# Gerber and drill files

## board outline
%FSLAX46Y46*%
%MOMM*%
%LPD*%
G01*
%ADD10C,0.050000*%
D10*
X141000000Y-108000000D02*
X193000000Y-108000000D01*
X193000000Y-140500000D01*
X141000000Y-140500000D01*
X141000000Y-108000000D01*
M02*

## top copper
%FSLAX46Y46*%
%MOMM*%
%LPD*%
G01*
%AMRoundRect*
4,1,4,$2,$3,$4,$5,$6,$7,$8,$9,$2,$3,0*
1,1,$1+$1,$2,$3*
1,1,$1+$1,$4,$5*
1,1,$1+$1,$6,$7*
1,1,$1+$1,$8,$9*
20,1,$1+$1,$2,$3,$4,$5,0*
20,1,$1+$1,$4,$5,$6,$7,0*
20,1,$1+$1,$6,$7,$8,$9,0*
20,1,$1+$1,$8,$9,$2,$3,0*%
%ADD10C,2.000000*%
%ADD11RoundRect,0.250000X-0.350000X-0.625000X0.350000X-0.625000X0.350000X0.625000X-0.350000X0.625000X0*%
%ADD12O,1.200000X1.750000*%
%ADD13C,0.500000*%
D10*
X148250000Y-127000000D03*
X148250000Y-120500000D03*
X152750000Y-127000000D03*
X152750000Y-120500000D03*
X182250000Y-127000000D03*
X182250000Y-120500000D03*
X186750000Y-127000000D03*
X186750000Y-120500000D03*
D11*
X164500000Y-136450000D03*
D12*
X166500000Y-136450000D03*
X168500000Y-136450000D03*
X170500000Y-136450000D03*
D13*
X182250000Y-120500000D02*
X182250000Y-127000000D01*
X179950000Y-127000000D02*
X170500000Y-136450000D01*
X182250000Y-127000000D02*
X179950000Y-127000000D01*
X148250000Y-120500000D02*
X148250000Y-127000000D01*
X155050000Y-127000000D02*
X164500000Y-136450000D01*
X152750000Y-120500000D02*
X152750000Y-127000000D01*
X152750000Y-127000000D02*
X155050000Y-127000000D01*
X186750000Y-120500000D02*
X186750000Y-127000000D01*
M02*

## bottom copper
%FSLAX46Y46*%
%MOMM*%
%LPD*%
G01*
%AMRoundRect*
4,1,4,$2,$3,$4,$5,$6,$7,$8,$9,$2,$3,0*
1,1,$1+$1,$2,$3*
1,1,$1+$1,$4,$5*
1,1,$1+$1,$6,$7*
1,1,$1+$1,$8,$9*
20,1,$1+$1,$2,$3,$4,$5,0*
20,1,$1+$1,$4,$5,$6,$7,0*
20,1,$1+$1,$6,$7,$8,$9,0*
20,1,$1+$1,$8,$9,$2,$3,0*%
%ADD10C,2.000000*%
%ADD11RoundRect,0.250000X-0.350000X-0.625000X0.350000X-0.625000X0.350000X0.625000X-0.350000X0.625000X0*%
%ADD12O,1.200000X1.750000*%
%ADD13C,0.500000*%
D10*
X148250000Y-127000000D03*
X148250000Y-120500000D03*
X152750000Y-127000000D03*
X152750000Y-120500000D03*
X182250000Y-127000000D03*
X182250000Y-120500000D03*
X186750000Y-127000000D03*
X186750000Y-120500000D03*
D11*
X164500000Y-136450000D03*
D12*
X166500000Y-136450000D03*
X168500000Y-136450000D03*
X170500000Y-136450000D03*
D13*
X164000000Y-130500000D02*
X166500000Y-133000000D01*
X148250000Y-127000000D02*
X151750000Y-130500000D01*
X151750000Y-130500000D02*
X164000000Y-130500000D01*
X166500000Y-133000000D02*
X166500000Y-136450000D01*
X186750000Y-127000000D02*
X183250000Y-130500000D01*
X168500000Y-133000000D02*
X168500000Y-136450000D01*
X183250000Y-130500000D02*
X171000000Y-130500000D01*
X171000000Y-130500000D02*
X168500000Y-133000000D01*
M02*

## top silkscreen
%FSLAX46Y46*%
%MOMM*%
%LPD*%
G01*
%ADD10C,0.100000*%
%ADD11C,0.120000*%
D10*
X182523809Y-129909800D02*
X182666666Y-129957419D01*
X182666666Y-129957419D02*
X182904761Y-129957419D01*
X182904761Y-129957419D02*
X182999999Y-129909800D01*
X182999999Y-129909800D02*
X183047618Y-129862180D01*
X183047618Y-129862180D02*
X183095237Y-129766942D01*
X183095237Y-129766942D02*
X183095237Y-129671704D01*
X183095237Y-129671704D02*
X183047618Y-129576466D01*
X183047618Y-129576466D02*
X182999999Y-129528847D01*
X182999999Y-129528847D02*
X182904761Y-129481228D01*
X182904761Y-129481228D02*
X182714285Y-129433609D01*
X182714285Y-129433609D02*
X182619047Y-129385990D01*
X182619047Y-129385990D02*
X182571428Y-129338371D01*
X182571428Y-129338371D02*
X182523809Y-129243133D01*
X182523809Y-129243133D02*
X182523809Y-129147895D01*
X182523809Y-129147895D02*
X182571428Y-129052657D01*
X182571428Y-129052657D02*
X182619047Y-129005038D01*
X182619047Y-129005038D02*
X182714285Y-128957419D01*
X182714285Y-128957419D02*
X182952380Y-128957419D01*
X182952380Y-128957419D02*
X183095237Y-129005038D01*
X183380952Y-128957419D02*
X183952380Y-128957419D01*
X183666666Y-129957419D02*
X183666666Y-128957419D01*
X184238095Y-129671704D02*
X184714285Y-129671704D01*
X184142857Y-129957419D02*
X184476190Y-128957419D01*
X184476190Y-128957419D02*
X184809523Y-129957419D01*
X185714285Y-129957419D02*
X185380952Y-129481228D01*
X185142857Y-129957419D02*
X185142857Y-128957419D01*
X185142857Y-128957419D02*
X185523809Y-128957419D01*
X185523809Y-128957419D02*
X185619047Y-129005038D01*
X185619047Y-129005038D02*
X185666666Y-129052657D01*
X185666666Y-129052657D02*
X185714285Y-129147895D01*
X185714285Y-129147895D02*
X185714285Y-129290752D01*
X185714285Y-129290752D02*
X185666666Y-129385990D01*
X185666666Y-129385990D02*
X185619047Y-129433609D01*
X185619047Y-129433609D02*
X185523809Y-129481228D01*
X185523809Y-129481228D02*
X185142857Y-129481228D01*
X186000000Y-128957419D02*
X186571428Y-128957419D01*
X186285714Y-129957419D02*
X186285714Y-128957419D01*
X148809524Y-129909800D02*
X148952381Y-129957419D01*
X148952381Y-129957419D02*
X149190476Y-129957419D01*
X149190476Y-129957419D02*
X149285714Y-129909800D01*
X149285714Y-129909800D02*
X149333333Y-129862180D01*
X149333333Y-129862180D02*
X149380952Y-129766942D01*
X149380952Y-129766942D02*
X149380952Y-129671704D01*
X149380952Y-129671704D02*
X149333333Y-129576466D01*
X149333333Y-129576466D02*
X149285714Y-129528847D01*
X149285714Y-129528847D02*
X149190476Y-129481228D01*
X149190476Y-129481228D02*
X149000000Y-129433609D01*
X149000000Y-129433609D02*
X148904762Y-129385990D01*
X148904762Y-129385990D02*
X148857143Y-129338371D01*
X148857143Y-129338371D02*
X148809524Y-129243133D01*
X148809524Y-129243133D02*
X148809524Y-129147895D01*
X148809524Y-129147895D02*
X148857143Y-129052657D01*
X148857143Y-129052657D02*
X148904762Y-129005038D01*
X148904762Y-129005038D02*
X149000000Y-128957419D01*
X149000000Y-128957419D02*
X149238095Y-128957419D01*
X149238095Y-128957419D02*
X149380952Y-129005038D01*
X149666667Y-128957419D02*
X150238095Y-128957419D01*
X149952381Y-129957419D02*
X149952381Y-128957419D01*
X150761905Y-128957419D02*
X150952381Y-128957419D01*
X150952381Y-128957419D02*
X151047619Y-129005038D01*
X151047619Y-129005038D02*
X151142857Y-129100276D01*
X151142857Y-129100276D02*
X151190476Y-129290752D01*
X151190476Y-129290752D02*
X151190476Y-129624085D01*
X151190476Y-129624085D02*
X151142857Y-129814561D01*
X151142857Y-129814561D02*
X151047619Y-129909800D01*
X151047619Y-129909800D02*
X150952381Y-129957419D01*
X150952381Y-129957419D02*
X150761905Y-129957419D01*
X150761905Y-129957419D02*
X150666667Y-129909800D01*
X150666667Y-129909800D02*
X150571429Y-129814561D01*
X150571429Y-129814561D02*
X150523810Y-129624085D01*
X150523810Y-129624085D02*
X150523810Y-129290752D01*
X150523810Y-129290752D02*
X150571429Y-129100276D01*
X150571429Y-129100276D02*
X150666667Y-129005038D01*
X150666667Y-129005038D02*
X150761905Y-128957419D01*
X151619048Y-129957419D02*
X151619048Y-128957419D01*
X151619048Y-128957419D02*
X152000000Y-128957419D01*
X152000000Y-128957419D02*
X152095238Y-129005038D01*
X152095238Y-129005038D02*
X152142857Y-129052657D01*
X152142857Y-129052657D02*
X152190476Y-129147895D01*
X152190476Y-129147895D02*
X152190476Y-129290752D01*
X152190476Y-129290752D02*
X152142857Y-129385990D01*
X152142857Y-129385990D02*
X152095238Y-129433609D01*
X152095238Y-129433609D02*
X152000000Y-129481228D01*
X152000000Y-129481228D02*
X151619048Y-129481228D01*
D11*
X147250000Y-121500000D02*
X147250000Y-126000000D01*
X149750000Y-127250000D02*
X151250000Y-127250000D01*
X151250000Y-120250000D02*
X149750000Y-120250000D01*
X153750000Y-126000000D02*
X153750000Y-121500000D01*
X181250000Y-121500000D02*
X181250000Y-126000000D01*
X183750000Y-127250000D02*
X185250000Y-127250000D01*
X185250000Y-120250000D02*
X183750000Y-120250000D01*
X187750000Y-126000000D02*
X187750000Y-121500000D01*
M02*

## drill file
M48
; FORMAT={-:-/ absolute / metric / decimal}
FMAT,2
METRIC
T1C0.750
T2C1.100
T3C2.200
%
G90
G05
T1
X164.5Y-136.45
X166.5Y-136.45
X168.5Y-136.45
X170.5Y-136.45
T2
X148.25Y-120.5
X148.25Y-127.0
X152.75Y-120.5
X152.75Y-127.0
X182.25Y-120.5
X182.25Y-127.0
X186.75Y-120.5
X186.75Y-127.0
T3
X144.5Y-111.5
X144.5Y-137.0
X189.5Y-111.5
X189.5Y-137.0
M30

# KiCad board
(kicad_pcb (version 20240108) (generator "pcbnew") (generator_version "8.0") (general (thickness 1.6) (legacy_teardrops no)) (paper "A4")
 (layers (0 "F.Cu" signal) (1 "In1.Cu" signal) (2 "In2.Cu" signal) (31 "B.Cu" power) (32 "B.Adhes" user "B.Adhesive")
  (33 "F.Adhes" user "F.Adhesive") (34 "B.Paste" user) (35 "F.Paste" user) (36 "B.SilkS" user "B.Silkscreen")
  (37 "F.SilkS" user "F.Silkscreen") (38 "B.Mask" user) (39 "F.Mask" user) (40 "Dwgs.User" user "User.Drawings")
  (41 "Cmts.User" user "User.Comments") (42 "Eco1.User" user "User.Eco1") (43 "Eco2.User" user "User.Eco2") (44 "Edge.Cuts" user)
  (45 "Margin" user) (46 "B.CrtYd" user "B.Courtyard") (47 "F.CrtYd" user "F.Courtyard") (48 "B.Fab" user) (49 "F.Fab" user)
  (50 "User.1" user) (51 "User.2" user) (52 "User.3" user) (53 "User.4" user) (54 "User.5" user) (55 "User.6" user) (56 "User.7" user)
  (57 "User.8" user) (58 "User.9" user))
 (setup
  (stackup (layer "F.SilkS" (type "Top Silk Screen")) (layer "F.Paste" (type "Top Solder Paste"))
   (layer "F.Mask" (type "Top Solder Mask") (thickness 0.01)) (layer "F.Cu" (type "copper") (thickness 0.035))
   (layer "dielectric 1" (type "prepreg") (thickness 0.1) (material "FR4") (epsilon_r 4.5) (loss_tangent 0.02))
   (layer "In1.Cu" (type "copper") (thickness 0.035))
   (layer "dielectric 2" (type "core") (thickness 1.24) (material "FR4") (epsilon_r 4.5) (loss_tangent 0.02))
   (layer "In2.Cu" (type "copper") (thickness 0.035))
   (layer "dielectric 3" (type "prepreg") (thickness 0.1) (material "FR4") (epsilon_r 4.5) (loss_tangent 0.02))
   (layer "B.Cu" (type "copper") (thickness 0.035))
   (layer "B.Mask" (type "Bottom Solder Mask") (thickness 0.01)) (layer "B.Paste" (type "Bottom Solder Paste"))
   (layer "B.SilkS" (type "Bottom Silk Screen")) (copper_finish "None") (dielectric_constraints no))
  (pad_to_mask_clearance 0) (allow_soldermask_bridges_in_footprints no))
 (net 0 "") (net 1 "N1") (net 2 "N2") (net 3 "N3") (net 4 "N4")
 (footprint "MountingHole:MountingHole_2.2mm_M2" (layer "F.Cu") (at 144.5 137)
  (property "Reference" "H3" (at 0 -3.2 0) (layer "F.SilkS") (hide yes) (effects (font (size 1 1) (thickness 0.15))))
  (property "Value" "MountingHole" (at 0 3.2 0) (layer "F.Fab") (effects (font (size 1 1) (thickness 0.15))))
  (pad "" np_thru_hole circle (at 0 0) (size 2.2 2.2) (drill 2.2) (layers "*.Cu" "*.Mask")))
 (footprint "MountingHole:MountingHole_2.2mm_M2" (layer "F.Cu") (at 189.5 137)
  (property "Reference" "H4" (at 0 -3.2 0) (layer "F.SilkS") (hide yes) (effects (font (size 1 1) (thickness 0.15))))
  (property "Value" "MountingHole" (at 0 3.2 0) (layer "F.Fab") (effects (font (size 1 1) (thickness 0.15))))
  (pad "" np_thru_hole circle (at 0 0) (size 2.2 2.2) (drill 2.2) (layers "*.Cu" "*.Mask")))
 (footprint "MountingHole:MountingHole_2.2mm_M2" (layer "F.Cu") (at 189.5 111.5)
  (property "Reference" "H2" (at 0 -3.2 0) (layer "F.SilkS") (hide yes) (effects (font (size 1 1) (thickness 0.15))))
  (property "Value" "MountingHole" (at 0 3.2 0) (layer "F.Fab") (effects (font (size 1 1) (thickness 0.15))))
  (pad "" np_thru_hole circle (at 0 0) (size 2.2 2.2) (drill 2.2) (layers "*.Cu" "*.Mask")))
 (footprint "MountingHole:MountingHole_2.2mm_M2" (layer "F.Cu") (at 144.5 111.5)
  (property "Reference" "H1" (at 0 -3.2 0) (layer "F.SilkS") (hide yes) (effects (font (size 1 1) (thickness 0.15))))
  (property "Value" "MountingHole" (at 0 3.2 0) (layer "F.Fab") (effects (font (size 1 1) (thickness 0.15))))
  (pad "" np_thru_hole circle (at 0 0) (size 2.2 2.2) (drill 2.2) (layers "*.Cu" "*.Mask")))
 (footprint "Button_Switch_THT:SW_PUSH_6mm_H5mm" (layer "F.Cu") (at 148.25 127 90)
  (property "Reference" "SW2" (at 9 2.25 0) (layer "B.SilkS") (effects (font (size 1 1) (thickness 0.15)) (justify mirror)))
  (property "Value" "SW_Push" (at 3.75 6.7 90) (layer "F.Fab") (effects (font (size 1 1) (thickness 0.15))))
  (fp_line (start 5.5 -1) (end 1 -1) (stroke (width 0.12) (type solid)) (layer "F.SilkS"))
  (fp_line (start -0.25 1.5) (end -0.25 3) (stroke (width 0.12) (type solid)) (layer "F.SilkS"))
  (fp_line (start 6.75 3) (end 6.75 1.5) (stroke (width 0.12) (type solid)) (layer "F.SilkS"))
  (fp_line (start 1 5.5) (end 5.5 5.5) (stroke (width 0.12) (type solid)) (layer "F.SilkS"))
  (pad "1" thru_hole circle (at 0 0 180) (size 2 2) (drill 1.1) (layers "*.Cu" "*.Mask") (remove_unused_layers no) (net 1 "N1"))
  (pad "1" thru_hole circle (at 6.5 0 180) (size 2 2) (drill 1.1) (layers "*.Cu" "*.Mask") (remove_unused_layers no) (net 1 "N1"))
  (pad "2" thru_hole circle (at 0 4.5 180) (size 2 2) (drill 1.1) (layers "*.Cu" "*.Mask") (remove_unused_layers no) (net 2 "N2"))
  (pad "2" thru_hole circle (at 6.5 4.5 180) (size 2 2) (drill 1.1) (layers "*.Cu" "*.Mask") (remove_unused_layers no) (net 2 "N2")))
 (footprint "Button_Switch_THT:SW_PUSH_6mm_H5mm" (layer "F.Cu") (at 182.25 127 90)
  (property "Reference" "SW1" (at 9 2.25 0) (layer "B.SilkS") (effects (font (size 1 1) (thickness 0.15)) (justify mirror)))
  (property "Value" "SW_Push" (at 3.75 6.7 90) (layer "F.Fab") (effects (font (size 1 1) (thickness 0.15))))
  (fp_line (start 5.5 -1) (end 1 -1) (stroke (width 0.12) (type solid)) (layer "F.SilkS"))
  (fp_line (start -0.25 1.5) (end -0.25 3) (stroke (width 0.12) (type solid)) (layer "F.SilkS"))
  (fp_line (start 6.75 3) (end 6.75 1.5) (stroke (width 0.12) (type solid)) (layer "F.SilkS"))
  (fp_line (start 1 5.5) (end 5.5 5.5) (stroke (width 0.12) (type solid)) (layer "F.SilkS"))
  (pad "1" thru_hole circle (at 0 0 180) (size 2 2) (drill 1.1) (layers "*.Cu" "*.Mask") (remove_unused_layers no) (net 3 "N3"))
  (pad "1" thru_hole circle (at 6.5 0 180) (size 2 2) (drill 1.1) (layers "*.Cu" "*.Mask") (remove_unused_layers no) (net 3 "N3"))
  (pad "2" thru_hole circle (at 0 4.5 180) (size 2 2) (drill 1.1) (layers "*.Cu" "*.Mask") (remove_unused_layers no) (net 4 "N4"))
  (pad "2" thru_hole circle (at 6.5 4.5 180) (size 2 2) (drill 1.1) (layers "*.Cu" "*.Mask") (remove_unused_layers no) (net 4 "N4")))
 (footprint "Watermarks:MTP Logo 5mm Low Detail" (layer "B.Cu") (at 179 135 180)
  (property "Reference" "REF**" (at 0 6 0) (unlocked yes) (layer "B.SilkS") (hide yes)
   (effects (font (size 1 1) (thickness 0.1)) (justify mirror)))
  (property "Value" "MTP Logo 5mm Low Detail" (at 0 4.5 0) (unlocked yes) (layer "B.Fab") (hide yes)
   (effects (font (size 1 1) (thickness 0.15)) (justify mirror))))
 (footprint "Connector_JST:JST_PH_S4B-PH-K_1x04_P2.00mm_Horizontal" (layer "B.Cu") (at 164.5 136.45)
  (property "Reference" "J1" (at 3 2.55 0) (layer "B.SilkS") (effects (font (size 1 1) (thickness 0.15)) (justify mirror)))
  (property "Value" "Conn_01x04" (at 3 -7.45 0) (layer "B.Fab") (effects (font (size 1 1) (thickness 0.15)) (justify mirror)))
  (pad "1" thru_hole roundrect (at 0 0) (size 1.2 1.75) (drill 0.75) (layers "*.Cu" "*.Mask") (remove_unused_layers no)
   (roundrect_rratio 0.208333) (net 2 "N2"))
  (pad "2" thru_hole oval (at 2 0) (size 1.2 1.75) (drill 0.75) (layers "*.Cu" "*.Mask") (remove_unused_layers no) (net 1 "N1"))
  (pad "3" thru_hole oval (at 4 0) (size 1.2 1.75) (drill 0.75) (layers "*.Cu" "*.Mask") (remove_unused_layers no) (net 4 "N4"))
  (pad "4" thru_hole oval (at 6 0) (size 1.2 1.75) (drill 0.75) (layers "*.Cu" "*.Mask") (remove_unused_layers no) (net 3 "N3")))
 (gr_rect (start 141 108) (end 193 140.5) (stroke (width 0.05) (type default)) (fill none) (layer "Edge.Cuts"))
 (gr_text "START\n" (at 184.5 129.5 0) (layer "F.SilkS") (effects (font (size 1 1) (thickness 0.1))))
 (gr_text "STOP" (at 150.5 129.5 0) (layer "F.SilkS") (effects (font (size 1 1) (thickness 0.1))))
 (segment (start 182.25 120.5) (end 182.25 127) (width 0.5) (layer "F.Cu") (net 3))
 (segment (start 179.95 127) (end 170.5 136.45) (width 0.5) (layer "F.Cu") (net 3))
 (segment (start 182.25 127) (end 179.95 127) (width 0.5) (layer "F.Cu") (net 3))
 (segment (start 148.25 120.5) (end 148.25 127) (width 0.5) (layer "F.Cu") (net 1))
 (segment (start 164 130.5) (end 166.5 133) (width 0.5) (layer "B.Cu") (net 1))
 (segment (start 148.25 127) (end 151.75 130.5) (width 0.5) (layer "B.Cu") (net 1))
 (segment (start 151.75 130.5) (end 164 130.5) (width 0.5) (layer "B.Cu") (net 1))
 (segment (start 166.5 133) (end 166.5 136.45) (width 0.5) (layer "B.Cu") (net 1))
 (segment (start 155.05 127) (end 164.5 136.45) (width 0.5) (layer "F.Cu") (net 2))
 (segment (start 152.75 120.5) (end 152.75 127) (width 0.5) (layer "F.Cu") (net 2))
 (segment (start 152.75 127) (end 155.05 127) (width 0.5) (layer "F.Cu") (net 2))
 (segment (start 186.75 120.5) (end 186.75 127) (width 0.5) (layer "F.Cu") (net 4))
 (segment (start 186.75 127) (end 183.25 130.5) (width 0.5) (layer "B.Cu") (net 4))
 (segment (start 168.5 133) (end 168.5 136.45) (width 0.5) (layer "B.Cu") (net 4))
 (segment (start 183.25 130.5) (end 171 130.5) (width 0.5) (layer "B.Cu") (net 4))
 (segment (start 171 130.5) (end 168.5 133) (width 0.5) (layer "B.Cu") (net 4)))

